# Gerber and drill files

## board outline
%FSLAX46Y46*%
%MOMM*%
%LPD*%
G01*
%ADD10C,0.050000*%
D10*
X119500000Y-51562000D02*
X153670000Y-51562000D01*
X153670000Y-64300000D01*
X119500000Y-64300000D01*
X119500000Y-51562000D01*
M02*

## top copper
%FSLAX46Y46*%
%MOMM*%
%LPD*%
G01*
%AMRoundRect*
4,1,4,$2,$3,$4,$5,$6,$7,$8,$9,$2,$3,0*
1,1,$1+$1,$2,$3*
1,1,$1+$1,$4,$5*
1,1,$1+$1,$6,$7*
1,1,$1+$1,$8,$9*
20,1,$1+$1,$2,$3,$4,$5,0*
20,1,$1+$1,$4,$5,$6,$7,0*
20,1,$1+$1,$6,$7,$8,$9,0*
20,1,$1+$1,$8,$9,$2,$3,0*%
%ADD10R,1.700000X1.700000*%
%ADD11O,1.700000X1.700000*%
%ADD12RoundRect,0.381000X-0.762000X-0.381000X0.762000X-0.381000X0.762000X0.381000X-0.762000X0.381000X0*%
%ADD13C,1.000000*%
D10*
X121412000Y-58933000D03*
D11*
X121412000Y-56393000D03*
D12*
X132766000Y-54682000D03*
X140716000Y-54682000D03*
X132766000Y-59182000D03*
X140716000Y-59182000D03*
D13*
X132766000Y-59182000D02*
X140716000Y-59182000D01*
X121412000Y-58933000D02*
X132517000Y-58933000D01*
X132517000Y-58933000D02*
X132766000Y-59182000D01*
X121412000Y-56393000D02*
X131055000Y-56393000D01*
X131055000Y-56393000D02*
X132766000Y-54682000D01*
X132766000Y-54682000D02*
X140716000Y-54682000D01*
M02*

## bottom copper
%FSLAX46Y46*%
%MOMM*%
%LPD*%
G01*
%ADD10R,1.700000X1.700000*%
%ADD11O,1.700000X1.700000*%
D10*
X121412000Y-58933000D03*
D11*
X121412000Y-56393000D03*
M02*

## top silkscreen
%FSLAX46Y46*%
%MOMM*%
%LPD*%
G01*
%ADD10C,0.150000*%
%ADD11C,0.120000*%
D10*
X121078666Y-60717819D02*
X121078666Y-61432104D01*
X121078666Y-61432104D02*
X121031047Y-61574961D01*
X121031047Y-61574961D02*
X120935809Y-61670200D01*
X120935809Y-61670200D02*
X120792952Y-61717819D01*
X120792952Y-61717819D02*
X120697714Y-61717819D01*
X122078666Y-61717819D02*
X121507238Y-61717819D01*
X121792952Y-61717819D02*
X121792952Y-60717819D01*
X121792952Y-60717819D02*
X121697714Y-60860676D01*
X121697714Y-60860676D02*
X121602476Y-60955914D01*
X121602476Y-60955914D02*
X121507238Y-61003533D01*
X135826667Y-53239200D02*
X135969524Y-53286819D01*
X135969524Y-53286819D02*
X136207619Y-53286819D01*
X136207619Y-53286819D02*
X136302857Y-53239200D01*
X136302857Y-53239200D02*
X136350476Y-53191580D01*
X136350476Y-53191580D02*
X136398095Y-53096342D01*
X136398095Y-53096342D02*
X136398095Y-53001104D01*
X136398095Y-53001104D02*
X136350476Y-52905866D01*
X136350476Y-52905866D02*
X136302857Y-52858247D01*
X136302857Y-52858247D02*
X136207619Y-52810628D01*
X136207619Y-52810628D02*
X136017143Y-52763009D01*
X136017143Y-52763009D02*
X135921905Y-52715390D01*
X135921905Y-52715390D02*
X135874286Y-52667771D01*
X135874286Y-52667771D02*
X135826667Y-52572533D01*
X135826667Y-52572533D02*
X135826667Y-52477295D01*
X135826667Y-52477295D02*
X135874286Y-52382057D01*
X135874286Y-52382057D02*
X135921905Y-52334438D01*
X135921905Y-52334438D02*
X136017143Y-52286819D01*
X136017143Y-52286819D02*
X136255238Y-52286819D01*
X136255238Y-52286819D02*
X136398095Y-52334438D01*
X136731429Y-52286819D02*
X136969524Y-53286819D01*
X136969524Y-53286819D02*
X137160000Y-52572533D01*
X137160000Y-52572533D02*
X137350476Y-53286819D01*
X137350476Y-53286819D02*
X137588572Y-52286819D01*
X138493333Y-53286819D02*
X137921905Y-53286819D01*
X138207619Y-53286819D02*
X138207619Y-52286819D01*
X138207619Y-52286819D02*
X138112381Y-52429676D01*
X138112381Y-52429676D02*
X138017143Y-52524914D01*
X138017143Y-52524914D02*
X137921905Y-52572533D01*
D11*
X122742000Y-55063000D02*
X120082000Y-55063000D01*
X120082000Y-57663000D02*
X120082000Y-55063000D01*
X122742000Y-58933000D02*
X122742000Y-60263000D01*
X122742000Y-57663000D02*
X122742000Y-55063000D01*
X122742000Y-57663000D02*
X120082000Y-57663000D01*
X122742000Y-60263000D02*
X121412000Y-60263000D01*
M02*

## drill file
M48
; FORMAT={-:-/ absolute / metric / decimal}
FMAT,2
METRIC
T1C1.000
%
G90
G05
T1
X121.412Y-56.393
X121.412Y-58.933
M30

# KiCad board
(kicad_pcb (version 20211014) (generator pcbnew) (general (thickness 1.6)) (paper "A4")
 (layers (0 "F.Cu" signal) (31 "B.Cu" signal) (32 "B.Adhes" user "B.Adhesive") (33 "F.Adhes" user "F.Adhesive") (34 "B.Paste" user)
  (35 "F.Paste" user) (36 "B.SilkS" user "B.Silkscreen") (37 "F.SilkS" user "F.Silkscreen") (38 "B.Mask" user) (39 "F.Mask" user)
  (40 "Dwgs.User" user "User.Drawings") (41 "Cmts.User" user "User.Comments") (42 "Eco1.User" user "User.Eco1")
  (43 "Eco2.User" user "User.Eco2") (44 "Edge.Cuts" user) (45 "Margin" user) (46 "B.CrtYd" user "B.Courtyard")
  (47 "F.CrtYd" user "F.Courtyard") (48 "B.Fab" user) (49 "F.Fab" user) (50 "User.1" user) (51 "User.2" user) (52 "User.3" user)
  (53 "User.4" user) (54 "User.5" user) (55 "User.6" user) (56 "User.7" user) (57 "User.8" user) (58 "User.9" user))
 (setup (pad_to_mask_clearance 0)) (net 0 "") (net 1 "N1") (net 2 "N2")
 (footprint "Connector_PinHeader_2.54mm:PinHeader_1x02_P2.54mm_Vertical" (layer "F.Cu") (at 121.412 58.933 180)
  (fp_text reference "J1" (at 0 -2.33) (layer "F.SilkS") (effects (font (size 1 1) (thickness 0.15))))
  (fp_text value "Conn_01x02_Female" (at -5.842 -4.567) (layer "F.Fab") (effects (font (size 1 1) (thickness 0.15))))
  (fp_line (start -1.33 3.87) (end 1.33 3.87) (layer "F.SilkS") (width 0.12))
  (fp_line (start 1.33 1.27) (end 1.33 3.87) (layer "F.SilkS") (width 0.12))
  (fp_line (start -1.33 0) (end -1.33 -1.33) (layer "F.SilkS") (width 0.12))
  (fp_line (start -1.33 1.27) (end -1.33 3.87) (layer "F.SilkS") (width 0.12))
  (fp_line (start -1.33 1.27) (end 1.33 1.27) (layer "F.SilkS") (width 0.12))
  (fp_line (start -1.33 -1.33) (end 0 -1.33) (layer "F.SilkS") (width 0.12))
  (pad "1" thru_hole rect (at 0 0 180) (size 1.7 1.7) (drill 1) (layers *.Cu *.Mask) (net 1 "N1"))
  (pad "2" thru_hole oval (at 0 2.54 180) (size 1.7 1.7) (drill 1) (layers *.Cu *.Mask) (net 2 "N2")))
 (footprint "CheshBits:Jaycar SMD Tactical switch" (layer "F.Cu") (at 137.466 49.982)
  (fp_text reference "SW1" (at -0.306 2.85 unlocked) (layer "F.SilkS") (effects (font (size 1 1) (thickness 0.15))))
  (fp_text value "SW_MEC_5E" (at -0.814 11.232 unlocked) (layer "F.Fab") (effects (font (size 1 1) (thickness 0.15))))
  (pad "1" smd roundrect (at -4.7 4.7) (size 2.286 1.524) (layers "F.Cu" "F.Paste" "F.Mask") (roundrect_rratio 0.25) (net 2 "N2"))
  (pad "2" smd roundrect (at 3.25 4.7) (size 2.286 1.524) (layers "F.Cu" "F.Paste" "F.Mask") (roundrect_rratio 0.25) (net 2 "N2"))
  (pad "3" smd roundrect (at -4.7 9.2) (size 2.286 1.524) (layers "F.Cu" "F.Paste" "F.Mask") (roundrect_rratio 0.25) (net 1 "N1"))
  (pad "4" smd roundrect (at 3.25 9.2) (size 2.286 1.524) (layers "F.Cu" "F.Paste" "F.Mask") (roundrect_rratio 0.25) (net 1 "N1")))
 (gr_rect (start 119.5 51.562) (end 153.67 64.3) (layer "Edge.Cuts") (width 0.05) (fill none))
 (segment (start 132.766 59.182) (end 140.716 59.182) (width 1) (layer "F.Cu") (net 1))
 (segment (start 121.412 58.933) (end 132.517 58.933) (width 1) (layer "F.Cu") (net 1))
 (segment (start 132.517 58.933) (end 132.766 59.182) (width 1) (layer "F.Cu") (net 1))
 (segment (start 121.412 56.393) (end 131.055 56.393) (width 1) (layer "F.Cu") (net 2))
 (segment (start 131.055 56.393) (end 132.766 54.682) (width 1) (layer "F.Cu") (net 2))
 (segment (start 132.766 54.682) (end 140.716 54.682) (width 1) (layer "F.Cu") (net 2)))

